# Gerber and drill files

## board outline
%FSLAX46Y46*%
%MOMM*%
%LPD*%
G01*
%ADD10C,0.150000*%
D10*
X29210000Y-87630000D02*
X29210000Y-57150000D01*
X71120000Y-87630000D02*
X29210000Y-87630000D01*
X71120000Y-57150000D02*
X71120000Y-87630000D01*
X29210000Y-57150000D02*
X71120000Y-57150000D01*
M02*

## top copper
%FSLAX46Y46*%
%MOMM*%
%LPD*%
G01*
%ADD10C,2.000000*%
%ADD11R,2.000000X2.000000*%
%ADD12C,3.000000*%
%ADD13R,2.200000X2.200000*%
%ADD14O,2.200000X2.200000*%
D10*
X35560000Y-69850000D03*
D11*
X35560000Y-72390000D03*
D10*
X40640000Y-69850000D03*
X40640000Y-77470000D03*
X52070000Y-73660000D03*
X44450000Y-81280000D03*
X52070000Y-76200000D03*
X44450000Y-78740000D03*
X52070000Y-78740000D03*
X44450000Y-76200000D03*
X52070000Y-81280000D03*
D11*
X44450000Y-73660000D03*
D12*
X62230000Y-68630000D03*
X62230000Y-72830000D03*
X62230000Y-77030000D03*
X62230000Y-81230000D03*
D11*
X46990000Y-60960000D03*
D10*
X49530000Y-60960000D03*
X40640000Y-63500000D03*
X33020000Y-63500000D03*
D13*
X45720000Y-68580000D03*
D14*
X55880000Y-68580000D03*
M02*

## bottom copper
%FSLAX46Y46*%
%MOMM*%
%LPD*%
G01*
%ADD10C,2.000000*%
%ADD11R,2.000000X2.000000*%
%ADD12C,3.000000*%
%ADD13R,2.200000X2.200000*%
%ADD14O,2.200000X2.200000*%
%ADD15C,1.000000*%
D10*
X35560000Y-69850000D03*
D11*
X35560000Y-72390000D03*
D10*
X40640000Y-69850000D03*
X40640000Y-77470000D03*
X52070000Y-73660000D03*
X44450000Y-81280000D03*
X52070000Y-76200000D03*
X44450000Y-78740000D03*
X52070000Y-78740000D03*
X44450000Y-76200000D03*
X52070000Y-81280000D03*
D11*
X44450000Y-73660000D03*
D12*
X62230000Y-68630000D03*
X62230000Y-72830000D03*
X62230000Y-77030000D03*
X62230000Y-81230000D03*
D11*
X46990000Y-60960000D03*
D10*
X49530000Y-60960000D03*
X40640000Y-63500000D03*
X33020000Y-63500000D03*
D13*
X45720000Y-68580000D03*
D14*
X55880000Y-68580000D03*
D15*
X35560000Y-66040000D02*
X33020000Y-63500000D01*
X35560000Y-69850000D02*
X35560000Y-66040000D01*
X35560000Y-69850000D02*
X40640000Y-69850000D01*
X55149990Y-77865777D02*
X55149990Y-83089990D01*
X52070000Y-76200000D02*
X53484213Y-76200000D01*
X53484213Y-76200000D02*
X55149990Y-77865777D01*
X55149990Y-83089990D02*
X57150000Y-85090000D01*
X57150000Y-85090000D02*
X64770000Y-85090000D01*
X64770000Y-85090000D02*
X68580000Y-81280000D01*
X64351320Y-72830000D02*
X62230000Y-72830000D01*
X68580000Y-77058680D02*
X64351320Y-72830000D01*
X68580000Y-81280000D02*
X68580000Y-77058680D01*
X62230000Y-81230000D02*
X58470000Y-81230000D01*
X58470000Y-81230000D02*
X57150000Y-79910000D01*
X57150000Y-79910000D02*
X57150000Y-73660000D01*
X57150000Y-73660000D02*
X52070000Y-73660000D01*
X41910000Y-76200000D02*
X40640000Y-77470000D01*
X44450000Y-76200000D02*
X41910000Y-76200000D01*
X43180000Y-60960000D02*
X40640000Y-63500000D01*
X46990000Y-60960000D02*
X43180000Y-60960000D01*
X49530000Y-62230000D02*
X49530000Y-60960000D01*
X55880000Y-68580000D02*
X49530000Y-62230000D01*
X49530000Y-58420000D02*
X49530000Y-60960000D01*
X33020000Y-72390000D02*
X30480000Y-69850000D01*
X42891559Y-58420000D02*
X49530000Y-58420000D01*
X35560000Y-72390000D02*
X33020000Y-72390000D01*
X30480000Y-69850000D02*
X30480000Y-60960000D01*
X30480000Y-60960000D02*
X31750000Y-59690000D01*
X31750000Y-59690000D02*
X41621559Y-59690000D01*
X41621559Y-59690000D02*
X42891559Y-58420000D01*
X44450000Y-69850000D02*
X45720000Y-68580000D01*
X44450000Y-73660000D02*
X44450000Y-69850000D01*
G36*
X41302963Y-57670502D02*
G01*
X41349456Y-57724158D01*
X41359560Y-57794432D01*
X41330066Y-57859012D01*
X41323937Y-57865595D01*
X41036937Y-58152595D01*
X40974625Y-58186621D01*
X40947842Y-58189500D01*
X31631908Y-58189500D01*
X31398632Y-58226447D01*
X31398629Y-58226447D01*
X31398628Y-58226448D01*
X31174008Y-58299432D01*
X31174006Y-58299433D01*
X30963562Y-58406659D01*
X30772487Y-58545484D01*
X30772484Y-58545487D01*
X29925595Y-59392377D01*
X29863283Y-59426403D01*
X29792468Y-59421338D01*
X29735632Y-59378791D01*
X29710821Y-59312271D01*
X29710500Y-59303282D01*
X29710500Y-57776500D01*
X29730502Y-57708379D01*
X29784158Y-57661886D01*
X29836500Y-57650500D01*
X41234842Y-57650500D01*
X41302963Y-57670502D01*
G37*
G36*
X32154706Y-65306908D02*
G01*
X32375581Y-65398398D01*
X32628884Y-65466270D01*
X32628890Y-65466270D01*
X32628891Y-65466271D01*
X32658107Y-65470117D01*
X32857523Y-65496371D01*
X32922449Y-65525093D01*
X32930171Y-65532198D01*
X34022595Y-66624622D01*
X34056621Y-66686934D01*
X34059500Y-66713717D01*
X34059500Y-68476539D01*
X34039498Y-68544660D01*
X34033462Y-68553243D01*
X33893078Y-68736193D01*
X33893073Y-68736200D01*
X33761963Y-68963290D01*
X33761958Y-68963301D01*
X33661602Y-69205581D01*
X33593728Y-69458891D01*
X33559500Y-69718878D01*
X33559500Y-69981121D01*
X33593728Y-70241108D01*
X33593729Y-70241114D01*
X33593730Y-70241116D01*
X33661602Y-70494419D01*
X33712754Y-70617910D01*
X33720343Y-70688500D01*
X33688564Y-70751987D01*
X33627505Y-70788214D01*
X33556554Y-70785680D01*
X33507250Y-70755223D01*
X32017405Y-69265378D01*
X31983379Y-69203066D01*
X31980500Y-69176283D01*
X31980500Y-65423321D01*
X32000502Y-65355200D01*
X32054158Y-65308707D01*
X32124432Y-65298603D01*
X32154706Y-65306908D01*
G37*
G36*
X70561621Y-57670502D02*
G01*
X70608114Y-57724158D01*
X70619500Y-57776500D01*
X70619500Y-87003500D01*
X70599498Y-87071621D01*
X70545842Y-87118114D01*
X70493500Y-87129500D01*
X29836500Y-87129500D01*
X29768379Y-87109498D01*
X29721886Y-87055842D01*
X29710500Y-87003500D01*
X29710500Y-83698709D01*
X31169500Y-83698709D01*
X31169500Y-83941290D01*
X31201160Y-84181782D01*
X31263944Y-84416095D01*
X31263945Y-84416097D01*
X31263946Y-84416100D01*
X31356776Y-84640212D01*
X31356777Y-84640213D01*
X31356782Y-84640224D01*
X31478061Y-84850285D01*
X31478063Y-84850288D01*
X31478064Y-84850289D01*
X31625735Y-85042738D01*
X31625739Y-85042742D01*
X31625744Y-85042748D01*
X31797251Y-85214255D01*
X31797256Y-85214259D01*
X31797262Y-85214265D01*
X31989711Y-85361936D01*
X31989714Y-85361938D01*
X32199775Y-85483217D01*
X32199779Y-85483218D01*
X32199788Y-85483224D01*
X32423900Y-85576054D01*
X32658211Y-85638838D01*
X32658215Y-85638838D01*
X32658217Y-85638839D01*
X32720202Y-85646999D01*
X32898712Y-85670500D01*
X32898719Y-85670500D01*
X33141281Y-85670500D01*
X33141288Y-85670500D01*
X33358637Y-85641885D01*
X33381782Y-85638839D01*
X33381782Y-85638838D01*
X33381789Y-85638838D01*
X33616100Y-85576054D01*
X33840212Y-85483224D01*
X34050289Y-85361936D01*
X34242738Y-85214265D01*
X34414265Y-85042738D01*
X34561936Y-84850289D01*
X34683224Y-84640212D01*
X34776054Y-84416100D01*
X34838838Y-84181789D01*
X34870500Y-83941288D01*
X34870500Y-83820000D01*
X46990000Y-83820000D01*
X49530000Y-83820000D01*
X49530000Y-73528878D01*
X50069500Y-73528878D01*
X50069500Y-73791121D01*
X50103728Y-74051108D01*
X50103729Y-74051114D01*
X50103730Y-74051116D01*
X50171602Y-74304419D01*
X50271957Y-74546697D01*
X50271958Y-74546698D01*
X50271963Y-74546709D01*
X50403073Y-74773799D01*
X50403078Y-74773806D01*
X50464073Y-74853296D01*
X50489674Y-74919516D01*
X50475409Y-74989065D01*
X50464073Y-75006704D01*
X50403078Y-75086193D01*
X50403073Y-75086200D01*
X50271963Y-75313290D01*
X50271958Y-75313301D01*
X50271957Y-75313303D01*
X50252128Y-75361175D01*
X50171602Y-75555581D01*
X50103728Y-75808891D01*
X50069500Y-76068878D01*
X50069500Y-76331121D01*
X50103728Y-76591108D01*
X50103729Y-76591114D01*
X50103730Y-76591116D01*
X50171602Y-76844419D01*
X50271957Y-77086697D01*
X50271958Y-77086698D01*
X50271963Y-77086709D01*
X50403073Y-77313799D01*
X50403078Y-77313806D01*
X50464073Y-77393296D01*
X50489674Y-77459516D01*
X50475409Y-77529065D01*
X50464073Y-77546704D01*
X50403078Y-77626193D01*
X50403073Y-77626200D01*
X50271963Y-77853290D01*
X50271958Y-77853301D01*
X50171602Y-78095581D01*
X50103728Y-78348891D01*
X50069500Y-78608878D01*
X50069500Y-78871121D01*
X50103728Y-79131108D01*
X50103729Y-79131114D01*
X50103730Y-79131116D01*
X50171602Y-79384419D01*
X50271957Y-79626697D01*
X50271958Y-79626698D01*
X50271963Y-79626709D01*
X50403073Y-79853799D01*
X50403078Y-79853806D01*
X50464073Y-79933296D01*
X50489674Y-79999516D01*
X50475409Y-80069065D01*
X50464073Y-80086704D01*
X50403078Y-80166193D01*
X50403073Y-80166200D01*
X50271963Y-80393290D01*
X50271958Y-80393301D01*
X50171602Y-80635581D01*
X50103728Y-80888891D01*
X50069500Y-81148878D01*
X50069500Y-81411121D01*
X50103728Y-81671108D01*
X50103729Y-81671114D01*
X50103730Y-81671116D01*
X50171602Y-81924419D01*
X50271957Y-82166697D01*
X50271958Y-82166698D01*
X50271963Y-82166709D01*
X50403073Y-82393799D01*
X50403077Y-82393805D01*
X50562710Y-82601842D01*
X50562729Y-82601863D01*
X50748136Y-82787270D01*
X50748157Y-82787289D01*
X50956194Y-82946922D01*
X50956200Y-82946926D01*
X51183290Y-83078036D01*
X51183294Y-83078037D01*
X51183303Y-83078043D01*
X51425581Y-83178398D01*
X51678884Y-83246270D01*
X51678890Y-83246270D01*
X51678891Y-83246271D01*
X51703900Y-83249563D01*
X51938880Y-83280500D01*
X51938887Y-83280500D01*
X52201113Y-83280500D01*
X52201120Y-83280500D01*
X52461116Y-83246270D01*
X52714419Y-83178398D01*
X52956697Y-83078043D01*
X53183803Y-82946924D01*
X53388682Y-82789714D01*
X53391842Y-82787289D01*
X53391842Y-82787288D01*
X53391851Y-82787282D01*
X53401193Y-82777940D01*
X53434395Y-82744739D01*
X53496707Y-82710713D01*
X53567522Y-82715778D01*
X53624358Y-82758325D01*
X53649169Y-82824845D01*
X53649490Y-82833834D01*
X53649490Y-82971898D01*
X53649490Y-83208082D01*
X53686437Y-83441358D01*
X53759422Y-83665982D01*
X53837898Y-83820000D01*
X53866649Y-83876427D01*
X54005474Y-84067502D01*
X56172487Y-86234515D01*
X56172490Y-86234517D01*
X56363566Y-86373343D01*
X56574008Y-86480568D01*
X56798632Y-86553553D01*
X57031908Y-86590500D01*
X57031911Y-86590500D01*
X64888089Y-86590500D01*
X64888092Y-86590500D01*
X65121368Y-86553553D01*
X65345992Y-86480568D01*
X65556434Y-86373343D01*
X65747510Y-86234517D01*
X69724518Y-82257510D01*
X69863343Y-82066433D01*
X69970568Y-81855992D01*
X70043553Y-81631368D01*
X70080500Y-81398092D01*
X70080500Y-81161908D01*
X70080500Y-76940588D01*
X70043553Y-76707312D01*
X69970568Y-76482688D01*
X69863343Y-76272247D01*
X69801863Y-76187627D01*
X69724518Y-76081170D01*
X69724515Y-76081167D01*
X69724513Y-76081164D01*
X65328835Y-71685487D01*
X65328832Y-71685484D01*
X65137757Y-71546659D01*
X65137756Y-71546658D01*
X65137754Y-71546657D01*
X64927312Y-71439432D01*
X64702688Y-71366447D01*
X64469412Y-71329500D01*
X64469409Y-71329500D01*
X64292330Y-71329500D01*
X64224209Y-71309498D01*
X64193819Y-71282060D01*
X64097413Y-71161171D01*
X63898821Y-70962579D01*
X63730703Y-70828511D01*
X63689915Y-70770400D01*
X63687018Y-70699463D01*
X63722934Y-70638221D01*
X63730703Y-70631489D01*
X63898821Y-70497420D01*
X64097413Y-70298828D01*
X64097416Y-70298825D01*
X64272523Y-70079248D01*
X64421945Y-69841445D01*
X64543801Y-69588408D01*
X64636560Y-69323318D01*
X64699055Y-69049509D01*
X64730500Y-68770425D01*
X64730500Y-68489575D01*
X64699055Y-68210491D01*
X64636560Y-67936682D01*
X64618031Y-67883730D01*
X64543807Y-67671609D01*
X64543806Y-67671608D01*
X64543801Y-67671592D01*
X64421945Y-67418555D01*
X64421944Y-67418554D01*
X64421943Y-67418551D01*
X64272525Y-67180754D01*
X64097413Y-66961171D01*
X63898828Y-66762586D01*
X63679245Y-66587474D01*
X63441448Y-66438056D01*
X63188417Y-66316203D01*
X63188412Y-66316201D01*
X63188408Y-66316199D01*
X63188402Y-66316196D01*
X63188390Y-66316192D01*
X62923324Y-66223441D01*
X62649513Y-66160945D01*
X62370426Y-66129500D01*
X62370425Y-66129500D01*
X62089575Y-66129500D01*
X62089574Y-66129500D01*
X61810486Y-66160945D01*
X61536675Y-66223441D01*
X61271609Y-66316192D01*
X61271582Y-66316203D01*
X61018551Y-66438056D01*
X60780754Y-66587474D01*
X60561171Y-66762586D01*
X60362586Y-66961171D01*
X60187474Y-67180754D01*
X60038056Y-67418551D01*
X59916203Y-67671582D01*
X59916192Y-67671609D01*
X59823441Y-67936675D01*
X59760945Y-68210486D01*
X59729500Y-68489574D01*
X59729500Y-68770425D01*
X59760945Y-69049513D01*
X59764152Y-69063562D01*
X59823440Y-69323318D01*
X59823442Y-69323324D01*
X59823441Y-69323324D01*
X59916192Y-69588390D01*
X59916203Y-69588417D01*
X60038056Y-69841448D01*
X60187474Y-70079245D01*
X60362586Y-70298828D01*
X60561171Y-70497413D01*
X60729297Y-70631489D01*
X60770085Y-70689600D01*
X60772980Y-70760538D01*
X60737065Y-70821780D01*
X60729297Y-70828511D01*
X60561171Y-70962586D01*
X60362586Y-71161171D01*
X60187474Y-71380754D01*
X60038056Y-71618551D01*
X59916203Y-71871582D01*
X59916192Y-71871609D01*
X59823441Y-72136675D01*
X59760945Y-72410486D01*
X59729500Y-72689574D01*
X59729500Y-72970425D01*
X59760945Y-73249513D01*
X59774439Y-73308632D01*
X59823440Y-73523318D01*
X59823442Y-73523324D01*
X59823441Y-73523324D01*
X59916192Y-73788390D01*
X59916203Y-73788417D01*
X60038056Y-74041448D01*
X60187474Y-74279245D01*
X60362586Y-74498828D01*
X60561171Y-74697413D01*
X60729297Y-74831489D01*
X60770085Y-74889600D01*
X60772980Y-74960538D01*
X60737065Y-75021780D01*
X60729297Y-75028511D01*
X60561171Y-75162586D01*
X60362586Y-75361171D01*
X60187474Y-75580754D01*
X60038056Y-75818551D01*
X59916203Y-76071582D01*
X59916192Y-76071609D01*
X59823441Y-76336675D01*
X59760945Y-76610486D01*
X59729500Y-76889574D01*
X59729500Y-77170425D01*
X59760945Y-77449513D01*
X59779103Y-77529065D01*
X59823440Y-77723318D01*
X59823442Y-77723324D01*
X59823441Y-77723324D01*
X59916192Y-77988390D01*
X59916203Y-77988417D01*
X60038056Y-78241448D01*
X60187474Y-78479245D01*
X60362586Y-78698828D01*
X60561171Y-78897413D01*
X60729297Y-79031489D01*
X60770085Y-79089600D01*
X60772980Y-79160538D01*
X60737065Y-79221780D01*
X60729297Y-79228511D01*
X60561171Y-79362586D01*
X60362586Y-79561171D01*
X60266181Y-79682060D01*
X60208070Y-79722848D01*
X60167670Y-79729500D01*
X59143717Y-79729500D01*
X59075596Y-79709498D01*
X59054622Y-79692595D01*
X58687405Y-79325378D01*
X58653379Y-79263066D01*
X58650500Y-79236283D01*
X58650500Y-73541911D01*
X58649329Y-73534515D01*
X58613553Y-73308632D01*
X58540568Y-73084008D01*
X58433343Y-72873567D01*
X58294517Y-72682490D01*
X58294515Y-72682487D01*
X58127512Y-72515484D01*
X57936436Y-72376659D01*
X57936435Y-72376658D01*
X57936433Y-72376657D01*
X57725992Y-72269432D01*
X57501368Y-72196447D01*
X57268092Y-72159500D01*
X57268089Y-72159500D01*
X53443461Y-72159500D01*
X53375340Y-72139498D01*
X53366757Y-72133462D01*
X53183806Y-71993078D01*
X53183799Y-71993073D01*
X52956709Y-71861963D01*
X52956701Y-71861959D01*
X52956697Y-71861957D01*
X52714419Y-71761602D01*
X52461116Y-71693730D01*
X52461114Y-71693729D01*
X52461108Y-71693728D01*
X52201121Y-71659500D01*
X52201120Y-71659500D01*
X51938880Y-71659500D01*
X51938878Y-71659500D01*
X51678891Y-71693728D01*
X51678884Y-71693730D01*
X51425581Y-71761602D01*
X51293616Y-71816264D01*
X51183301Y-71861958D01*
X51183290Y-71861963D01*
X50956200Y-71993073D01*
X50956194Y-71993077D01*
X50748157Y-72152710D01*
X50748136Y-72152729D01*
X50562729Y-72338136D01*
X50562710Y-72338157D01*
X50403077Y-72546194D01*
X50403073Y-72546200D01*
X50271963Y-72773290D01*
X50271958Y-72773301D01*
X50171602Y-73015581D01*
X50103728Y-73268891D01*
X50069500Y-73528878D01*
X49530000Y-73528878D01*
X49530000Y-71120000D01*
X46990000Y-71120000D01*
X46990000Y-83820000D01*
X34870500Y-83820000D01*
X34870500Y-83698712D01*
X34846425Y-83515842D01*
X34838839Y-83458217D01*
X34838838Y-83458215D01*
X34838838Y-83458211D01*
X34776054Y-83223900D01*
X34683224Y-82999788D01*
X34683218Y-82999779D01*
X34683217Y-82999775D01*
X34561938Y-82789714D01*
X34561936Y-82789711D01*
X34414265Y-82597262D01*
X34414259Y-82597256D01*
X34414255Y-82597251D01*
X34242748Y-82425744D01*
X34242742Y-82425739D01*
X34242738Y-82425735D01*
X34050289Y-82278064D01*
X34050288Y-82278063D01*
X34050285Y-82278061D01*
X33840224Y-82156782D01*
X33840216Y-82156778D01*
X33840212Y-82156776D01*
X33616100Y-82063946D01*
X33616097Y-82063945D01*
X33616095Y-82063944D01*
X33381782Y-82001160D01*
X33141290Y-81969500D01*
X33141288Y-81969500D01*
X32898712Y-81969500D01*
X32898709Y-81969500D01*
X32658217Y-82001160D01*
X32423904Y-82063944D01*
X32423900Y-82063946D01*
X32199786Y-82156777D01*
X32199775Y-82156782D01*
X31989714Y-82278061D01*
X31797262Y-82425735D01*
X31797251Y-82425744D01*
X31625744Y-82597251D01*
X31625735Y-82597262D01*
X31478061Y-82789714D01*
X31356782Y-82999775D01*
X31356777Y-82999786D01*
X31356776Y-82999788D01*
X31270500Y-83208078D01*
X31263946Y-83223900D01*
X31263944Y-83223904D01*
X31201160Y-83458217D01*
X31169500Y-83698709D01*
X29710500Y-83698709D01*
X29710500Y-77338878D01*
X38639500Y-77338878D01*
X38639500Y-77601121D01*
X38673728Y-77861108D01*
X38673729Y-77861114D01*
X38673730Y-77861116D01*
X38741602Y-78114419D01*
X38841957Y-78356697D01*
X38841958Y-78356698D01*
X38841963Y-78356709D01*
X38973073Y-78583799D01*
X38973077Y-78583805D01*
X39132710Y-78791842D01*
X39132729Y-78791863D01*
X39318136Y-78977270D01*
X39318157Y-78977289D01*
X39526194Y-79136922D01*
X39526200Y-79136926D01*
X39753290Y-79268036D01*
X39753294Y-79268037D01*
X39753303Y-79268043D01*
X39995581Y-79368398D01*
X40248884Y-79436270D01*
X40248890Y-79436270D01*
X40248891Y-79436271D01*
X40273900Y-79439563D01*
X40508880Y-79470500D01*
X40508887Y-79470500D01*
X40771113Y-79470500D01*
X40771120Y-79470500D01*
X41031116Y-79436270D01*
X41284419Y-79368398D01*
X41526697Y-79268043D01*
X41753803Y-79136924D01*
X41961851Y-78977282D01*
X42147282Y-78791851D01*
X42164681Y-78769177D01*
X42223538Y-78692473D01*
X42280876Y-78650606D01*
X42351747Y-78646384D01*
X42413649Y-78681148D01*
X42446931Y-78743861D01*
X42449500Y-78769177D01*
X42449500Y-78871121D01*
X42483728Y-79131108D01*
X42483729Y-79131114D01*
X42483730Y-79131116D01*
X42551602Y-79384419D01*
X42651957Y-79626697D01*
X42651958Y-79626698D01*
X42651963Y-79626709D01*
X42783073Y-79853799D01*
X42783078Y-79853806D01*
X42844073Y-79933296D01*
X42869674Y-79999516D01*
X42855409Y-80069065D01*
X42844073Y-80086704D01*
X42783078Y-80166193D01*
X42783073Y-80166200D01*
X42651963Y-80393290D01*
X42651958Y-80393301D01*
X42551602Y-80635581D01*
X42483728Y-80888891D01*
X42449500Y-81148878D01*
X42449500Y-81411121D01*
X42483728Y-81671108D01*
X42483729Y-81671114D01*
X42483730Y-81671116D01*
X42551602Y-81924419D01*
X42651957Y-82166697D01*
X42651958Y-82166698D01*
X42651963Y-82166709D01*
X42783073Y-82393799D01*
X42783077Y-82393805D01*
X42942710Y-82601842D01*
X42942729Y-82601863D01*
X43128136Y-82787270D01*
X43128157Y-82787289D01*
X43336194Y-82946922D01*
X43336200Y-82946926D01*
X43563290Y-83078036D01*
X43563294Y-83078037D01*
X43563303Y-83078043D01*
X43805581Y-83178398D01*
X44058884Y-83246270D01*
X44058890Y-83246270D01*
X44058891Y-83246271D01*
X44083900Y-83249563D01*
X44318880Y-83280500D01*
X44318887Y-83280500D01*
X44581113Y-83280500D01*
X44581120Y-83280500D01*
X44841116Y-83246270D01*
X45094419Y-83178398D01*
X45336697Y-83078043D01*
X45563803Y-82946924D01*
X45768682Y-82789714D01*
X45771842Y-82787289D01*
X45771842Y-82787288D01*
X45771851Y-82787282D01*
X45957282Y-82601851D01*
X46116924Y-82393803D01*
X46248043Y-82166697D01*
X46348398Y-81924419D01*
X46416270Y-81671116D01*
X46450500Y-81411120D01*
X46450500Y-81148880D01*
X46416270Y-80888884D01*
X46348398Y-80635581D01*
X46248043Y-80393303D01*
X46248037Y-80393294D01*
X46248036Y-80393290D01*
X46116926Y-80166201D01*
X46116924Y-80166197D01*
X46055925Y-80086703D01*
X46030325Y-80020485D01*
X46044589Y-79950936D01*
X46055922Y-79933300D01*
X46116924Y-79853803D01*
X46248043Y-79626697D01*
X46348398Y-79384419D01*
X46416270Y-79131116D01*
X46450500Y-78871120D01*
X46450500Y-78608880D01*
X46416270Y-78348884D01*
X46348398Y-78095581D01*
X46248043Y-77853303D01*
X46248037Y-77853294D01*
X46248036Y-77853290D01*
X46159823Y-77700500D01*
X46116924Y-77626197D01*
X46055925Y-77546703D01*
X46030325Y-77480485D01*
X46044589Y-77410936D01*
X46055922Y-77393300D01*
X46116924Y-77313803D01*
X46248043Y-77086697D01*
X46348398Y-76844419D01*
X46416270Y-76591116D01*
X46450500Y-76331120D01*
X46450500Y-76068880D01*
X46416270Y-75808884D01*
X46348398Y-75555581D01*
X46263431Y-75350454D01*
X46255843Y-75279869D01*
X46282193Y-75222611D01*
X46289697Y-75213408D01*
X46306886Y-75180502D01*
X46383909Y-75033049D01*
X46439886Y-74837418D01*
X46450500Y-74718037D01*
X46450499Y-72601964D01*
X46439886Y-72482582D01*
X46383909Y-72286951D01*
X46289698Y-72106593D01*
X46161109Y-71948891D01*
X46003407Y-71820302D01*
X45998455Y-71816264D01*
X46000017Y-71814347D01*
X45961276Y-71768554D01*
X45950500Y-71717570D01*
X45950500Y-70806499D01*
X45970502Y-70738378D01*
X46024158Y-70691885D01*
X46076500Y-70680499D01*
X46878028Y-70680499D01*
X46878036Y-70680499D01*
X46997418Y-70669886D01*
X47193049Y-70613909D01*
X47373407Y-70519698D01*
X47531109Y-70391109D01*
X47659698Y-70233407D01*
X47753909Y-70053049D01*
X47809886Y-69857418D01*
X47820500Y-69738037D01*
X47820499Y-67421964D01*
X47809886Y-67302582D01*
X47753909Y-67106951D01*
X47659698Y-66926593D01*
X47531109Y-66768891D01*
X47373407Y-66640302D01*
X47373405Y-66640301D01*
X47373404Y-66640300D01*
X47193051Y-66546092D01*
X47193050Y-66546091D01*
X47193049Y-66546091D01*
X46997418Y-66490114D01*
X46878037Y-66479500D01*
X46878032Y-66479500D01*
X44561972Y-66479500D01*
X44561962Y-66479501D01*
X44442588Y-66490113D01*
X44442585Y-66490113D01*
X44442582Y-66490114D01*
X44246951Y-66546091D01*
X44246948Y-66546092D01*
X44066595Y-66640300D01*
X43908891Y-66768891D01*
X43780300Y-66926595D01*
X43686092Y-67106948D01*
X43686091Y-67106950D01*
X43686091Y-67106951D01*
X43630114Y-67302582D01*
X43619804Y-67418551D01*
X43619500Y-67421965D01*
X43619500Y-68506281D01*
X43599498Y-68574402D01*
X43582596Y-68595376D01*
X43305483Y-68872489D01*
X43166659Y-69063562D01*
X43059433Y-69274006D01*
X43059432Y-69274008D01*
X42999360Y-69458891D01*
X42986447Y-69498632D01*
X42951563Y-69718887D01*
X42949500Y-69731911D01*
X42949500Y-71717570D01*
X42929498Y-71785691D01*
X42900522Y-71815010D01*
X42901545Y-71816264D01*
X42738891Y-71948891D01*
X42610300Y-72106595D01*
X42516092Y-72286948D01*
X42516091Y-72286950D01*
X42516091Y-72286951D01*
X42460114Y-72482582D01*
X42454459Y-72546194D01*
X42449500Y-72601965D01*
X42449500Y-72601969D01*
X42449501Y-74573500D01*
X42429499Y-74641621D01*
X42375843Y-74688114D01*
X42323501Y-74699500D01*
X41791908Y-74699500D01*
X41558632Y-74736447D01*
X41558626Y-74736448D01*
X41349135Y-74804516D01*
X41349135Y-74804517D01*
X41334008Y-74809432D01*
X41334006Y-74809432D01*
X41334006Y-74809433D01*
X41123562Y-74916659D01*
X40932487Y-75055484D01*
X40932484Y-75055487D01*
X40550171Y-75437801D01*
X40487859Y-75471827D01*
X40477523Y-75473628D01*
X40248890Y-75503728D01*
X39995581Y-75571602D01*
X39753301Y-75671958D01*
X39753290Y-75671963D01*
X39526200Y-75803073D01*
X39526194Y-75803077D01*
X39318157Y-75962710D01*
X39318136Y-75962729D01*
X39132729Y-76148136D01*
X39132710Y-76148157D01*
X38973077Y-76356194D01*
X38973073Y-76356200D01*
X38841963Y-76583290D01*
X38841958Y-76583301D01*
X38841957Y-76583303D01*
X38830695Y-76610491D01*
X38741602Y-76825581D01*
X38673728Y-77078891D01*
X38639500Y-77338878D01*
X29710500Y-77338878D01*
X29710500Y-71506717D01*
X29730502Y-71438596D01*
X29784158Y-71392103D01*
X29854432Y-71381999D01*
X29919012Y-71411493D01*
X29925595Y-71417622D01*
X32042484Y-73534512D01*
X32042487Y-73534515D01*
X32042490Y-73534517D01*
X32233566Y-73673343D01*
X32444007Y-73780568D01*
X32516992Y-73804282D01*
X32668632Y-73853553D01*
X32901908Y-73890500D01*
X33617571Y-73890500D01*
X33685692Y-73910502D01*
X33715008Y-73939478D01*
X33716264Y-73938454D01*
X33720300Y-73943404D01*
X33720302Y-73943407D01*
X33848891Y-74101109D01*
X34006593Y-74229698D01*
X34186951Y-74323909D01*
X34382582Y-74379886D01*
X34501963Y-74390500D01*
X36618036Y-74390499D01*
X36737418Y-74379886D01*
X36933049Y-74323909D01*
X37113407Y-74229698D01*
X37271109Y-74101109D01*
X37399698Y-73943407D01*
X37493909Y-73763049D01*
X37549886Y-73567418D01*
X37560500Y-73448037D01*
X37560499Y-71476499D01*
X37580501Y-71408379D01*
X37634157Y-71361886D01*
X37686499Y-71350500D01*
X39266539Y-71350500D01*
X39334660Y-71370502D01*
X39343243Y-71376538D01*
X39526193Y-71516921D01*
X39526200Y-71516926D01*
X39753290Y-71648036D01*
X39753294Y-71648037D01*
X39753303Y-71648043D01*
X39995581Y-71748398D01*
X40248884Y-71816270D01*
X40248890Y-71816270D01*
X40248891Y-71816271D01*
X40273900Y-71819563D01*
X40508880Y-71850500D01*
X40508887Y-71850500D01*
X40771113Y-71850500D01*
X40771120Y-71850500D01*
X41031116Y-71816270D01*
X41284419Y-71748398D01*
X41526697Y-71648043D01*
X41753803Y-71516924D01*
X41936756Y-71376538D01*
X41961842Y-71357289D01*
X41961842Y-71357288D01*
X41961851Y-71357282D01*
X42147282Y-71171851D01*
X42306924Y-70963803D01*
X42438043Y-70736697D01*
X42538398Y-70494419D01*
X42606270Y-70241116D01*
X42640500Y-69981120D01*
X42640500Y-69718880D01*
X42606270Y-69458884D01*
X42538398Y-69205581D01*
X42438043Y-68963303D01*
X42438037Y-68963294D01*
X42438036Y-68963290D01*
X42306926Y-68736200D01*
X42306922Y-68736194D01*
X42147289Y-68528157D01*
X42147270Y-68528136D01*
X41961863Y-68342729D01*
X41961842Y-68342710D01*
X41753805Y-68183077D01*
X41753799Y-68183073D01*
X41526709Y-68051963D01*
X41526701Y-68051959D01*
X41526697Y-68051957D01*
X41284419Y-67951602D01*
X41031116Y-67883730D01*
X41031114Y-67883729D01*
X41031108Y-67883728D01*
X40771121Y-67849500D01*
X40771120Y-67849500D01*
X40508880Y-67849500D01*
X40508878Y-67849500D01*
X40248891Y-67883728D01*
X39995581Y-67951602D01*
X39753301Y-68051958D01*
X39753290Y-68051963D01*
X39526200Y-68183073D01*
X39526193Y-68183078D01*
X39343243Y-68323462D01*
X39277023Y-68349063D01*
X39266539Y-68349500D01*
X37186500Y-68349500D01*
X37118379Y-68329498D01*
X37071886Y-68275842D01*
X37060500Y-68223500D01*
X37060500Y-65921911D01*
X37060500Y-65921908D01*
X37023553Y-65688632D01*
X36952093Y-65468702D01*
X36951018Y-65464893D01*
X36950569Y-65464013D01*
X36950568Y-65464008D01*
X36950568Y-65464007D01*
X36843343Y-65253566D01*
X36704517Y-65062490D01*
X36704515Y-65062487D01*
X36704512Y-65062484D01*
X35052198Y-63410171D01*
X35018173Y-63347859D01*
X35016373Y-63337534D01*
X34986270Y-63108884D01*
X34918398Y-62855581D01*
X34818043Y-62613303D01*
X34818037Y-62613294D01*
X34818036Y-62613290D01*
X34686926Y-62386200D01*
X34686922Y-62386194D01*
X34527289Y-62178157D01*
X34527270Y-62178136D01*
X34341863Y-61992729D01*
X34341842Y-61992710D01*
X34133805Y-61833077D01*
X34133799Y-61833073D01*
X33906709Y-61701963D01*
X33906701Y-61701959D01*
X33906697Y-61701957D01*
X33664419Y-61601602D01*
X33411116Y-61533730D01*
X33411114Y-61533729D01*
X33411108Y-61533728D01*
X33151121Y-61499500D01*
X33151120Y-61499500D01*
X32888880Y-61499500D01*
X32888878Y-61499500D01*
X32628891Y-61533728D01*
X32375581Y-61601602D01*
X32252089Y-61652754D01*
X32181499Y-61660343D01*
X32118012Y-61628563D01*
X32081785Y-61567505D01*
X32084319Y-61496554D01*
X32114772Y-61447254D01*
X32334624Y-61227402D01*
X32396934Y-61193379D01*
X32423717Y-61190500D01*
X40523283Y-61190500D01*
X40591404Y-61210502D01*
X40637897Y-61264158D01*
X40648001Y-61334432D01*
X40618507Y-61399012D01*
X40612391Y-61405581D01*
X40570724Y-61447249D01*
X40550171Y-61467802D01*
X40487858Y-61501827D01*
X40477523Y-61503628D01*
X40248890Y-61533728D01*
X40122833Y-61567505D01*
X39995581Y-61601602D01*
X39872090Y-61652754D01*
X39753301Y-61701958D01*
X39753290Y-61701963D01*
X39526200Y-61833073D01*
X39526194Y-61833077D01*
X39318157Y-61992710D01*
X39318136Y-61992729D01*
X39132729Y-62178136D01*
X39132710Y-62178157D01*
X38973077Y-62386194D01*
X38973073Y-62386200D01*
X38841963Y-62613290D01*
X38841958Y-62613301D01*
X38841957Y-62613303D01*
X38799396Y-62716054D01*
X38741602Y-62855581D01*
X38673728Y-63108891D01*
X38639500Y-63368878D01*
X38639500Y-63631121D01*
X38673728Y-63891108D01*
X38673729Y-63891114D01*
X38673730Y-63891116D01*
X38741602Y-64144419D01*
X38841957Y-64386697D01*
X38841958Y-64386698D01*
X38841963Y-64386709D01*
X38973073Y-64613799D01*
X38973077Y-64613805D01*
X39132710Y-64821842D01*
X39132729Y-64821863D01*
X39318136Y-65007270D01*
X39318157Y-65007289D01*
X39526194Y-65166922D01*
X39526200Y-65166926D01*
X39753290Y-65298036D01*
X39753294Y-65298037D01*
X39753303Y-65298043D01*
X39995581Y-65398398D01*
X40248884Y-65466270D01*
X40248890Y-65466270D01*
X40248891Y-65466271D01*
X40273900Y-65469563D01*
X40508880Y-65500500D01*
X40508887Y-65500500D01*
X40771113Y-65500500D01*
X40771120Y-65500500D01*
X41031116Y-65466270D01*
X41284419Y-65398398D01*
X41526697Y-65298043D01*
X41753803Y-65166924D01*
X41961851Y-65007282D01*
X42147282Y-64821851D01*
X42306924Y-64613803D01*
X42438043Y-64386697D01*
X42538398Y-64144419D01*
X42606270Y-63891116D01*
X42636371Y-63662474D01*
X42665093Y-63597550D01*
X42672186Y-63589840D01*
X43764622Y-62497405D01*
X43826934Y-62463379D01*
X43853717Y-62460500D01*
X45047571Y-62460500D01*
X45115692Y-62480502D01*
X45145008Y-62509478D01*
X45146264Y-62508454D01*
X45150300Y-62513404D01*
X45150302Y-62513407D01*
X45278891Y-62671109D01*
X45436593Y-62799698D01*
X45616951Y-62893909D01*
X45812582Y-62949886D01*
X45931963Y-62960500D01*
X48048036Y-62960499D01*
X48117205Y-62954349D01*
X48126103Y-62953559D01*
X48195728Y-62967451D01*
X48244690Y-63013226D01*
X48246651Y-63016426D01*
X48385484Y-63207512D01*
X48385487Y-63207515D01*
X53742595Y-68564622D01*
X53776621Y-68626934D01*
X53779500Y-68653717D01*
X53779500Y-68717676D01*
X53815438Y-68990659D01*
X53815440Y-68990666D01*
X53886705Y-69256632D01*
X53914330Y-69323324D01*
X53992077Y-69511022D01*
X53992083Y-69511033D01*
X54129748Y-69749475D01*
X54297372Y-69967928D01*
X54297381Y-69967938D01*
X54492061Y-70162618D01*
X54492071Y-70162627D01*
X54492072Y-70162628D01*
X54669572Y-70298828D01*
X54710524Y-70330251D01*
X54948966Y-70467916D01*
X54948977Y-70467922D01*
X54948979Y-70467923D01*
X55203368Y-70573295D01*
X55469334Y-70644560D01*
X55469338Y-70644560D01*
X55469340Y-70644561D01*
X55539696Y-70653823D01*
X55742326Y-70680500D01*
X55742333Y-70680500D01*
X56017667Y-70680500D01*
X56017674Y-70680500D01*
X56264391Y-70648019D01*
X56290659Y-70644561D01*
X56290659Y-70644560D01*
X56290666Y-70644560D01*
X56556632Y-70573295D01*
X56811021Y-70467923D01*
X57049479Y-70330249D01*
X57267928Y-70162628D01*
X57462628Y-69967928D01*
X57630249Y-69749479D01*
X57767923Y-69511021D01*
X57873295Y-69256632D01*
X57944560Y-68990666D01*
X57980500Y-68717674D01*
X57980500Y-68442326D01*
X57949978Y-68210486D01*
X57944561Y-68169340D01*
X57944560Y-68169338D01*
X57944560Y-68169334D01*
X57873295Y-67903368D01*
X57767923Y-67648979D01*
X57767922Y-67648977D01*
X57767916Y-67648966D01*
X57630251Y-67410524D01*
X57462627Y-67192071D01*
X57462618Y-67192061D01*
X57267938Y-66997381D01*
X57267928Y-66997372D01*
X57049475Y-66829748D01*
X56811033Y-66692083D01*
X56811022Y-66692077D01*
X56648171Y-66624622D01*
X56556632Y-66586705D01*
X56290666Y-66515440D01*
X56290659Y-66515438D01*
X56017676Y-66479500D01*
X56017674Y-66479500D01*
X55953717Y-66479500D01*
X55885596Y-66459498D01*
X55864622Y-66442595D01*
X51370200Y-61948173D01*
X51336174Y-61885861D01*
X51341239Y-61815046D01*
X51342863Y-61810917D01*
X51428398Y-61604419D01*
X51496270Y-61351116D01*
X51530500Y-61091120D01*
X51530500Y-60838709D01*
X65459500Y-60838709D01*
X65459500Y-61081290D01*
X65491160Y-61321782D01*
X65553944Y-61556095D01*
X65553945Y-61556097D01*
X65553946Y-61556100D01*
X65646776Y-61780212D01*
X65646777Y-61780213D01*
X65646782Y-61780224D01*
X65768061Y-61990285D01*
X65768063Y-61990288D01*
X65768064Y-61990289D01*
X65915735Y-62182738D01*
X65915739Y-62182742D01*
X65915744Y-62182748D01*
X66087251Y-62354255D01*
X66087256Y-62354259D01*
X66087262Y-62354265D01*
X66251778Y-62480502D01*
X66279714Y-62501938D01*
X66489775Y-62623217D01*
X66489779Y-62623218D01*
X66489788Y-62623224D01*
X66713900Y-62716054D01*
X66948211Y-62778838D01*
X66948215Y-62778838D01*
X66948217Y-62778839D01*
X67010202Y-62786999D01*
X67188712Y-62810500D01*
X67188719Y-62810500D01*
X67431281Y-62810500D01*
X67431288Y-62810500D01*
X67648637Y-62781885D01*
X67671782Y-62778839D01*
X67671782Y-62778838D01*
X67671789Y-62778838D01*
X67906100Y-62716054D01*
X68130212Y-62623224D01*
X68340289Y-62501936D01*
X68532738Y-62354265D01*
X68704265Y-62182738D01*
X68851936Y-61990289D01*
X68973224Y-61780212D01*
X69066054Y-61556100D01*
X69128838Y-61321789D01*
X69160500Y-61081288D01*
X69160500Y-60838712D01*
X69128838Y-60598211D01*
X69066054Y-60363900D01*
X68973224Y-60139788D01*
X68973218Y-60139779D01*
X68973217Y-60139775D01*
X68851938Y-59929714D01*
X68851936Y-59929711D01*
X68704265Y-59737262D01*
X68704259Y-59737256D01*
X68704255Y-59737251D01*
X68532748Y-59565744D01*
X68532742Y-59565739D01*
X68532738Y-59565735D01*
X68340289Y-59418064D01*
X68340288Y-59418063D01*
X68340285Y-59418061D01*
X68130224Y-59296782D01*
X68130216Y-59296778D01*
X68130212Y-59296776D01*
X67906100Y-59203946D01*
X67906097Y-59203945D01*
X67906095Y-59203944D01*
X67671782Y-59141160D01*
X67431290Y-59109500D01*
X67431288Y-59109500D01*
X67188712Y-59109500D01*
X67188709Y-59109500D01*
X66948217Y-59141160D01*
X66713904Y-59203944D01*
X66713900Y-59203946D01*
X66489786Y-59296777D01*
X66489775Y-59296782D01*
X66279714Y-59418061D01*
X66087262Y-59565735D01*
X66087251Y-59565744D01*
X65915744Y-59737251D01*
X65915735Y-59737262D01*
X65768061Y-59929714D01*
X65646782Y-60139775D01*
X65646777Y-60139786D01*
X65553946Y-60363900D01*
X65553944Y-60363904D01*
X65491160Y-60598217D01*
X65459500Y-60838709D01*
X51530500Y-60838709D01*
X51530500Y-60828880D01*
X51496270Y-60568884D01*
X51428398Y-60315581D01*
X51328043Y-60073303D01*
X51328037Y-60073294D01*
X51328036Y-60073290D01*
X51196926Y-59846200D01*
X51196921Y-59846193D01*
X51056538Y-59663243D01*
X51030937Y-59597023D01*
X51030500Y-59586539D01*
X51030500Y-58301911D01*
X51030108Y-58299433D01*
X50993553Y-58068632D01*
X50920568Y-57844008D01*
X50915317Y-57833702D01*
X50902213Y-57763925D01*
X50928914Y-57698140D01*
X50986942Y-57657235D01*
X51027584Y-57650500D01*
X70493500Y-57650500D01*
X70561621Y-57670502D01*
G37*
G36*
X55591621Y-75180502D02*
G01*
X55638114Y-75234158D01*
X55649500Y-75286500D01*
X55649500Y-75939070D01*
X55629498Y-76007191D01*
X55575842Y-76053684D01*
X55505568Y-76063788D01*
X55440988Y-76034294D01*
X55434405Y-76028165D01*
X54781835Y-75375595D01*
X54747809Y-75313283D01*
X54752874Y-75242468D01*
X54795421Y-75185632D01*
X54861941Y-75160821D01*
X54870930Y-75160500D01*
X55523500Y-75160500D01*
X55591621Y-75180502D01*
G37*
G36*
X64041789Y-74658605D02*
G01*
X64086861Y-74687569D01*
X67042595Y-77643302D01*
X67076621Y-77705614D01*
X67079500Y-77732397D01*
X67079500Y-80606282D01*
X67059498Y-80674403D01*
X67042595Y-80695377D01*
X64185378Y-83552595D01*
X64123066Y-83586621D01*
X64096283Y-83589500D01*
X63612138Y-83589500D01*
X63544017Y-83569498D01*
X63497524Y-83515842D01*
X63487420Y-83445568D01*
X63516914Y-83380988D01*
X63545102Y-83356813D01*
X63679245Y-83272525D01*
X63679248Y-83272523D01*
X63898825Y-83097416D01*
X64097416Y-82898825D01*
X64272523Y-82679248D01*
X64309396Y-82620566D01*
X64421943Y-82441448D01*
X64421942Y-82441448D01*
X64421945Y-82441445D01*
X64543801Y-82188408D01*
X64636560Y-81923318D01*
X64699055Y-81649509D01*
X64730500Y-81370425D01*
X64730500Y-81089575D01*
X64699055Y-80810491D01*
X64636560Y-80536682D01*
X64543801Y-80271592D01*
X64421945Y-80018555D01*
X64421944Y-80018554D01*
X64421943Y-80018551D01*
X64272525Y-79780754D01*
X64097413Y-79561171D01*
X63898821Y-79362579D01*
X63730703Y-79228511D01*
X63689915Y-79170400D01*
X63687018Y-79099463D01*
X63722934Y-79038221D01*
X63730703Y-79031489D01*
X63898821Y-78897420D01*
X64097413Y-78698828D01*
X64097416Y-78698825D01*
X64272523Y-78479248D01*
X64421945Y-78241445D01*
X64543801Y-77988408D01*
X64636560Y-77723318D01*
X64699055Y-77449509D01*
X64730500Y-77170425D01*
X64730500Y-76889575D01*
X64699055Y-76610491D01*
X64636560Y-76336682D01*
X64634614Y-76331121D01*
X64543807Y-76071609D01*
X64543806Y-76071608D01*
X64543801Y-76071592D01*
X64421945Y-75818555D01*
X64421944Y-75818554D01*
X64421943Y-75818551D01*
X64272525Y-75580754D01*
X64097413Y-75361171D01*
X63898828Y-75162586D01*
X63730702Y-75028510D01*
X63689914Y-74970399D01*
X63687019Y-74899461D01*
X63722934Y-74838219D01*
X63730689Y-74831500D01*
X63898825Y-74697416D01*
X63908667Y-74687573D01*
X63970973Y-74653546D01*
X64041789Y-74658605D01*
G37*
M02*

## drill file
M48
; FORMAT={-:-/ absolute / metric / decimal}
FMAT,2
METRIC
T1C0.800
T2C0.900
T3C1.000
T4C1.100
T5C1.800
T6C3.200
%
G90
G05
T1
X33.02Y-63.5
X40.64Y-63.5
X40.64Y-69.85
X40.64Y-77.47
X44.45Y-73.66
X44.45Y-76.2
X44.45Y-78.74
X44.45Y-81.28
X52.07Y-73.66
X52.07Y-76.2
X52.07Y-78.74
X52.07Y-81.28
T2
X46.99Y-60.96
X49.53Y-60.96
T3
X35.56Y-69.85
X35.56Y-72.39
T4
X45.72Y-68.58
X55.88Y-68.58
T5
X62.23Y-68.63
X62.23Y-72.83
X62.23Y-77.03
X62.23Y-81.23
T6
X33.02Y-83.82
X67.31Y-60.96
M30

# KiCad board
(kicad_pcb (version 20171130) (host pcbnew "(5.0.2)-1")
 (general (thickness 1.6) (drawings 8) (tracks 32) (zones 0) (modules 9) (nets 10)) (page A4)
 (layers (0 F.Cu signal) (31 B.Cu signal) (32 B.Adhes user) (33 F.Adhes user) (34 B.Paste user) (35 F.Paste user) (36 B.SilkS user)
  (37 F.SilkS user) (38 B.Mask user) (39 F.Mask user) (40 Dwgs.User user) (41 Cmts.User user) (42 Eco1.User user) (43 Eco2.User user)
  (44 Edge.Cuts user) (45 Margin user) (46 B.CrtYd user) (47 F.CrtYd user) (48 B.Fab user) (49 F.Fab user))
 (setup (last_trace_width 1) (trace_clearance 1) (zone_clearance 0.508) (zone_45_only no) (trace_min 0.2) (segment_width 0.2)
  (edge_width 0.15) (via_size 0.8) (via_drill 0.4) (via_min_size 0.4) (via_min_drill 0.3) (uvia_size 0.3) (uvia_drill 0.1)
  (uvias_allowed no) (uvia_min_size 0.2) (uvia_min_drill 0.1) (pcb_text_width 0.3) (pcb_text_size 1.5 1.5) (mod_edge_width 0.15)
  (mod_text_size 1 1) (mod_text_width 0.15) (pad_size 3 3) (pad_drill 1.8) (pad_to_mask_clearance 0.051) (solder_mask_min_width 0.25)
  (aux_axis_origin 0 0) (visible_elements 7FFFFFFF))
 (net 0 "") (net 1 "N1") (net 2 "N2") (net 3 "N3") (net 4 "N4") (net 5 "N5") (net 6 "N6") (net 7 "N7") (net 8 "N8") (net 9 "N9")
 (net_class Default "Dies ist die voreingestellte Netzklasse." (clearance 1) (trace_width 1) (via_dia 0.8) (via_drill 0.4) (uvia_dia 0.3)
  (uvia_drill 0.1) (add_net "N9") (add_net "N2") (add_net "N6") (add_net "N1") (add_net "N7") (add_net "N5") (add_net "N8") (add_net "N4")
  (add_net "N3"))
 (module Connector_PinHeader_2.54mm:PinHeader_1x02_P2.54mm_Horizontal (layer F.Cu) (at 35.56 72.39 180)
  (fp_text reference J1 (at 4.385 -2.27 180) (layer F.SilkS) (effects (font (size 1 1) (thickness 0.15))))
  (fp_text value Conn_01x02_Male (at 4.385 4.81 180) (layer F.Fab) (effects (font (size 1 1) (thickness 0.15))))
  (pad 2 thru_hole circle (at 0 2.54 180) (size 2 2) (drill 1) (layers *.Cu *.Mask) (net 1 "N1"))
  (pad 1 thru_hole rect (at 0 0 180) (size 2 2) (drill 1) (layers *.Cu *.Mask) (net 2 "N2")))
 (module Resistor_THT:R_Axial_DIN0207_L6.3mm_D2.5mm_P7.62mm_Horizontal (layer F.Cu) (at 40.64 77.47 90)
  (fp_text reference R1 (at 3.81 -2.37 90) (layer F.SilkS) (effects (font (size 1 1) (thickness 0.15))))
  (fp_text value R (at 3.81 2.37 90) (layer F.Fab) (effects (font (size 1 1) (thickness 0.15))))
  (pad 2 thru_hole circle (at 7.62 0 90) (size 2 2) (drill 0.8) (layers *.Cu *.Mask) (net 1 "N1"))
  (pad 1 thru_hole circle (at 0 0 90) (size 2 2) (drill 0.8) (layers *.Cu *.Mask) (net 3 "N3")))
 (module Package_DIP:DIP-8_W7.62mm (layer F.Cu) (at 44.45 73.66)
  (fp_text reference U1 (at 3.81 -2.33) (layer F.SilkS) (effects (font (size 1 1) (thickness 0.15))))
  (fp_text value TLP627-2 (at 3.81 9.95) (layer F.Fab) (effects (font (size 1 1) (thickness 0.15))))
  (pad 8 thru_hole circle (at 7.62 0) (size 2 2) (drill 0.8) (layers *.Cu *.Mask) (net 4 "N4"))
  (pad 4 thru_hole circle (at 0 7.62) (size 2 2) (drill 0.8) (layers *.Cu *.Mask))
  (pad 7 thru_hole circle (at 7.62 2.54) (size 2 2) (drill 0.8) (layers *.Cu *.Mask) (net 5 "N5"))
  (pad 3 thru_hole circle (at 0 5.08) (size 2 2) (drill 0.8) (layers *.Cu *.Mask))
  (pad 6 thru_hole circle (at 7.62 5.08) (size 2 2) (drill 0.8) (layers *.Cu *.Mask))
  (pad 2 thru_hole circle (at 0 2.54) (size 2 2) (drill 0.8) (layers *.Cu *.Mask) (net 3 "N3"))
  (pad 5 thru_hole circle (at 7.62 7.62) (size 2 2) (drill 0.8) (layers *.Cu *.Mask))
  (pad 1 thru_hole rect (at 0 0) (size 2 2) (drill 0.8) (layers *.Cu *.Mask) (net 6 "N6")))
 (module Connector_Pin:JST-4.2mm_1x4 (layer F.Cu) (at 62.23 74.93 270)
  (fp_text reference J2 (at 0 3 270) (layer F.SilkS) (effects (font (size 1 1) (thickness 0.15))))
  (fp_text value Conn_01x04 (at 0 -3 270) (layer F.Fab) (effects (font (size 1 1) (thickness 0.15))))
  (pad 1 thru_hole circle (at -6.3 0 270) (size 3 3) (drill 1.8) (layers *.Cu *.Mask) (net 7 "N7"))
  (pad 2 thru_hole circle (at -2.1 0 270) (size 3 3) (drill 1.8) (layers *.Cu *.Mask) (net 5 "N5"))
  (pad 3 thru_hole circle (at 2.1 0 270) (size 3 3) (drill 1.8) (layers *.Cu *.Mask) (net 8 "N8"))
  (pad 4 thru_hole circle (at 6.3 0 270) (size 3 3) (drill 1.8) (layers *.Cu *.Mask) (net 4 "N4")))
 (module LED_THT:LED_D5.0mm (layer F.Cu) (at 46.99 60.96)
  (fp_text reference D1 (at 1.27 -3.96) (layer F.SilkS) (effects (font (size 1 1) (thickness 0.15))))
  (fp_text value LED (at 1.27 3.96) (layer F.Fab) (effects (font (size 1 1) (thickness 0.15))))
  (pad 1 thru_hole rect (at 0 0) (size 2 2) (drill 0.9) (layers *.Cu *.Mask) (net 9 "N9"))
  (pad 2 thru_hole circle (at 2.54 0) (size 2 2) (drill 0.9) (layers *.Cu *.Mask) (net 2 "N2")))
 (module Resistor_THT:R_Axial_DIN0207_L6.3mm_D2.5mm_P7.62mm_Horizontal (layer F.Cu) (at 40.64 63.5 180)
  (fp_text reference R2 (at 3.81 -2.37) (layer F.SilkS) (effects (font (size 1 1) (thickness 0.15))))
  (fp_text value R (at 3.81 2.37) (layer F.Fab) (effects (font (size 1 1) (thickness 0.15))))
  (pad 1 thru_hole circle (at 0 0 180) (size 2 2) (drill 0.8) (layers *.Cu *.Mask) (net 9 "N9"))
  (pad 2 thru_hole circle (at 7.62 0 180) (size 2 2) (drill 0.8) (layers *.Cu *.Mask) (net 1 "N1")))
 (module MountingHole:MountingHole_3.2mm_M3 (layer F.Cu) (at 33.02 83.82)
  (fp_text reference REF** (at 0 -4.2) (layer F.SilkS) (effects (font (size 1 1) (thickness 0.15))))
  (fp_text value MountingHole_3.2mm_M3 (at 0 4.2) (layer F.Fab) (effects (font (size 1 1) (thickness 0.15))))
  (pad 1 np_thru_hole circle (at 0 0) (size 3.2 3.2) (drill 3.2) (layers *.Cu *.Mask)))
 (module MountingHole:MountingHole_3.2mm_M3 (layer F.Cu) (at 67.31 60.96)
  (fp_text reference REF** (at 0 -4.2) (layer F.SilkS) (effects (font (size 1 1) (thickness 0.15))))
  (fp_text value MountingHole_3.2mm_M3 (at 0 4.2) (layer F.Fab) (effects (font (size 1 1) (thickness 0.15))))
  (pad 1 np_thru_hole circle (at 0 0) (size 3.2 3.2) (drill 3.2) (layers *.Cu *.Mask)))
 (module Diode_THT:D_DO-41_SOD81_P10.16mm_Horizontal (layer F.Cu) (at 45.72 68.58)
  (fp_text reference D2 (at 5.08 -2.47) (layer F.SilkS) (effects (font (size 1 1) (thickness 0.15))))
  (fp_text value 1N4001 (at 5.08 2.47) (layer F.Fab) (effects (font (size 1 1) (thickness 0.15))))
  (pad 1 thru_hole rect (at 0 0) (size 2.2 2.2) (drill 1.1) (layers *.Cu *.Mask) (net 6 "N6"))
  (pad 2 thru_hole oval (at 10.16 0) (size 2.2 2.2) (drill 1.1) (layers *.Cu *.Mask) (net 2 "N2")))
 (gr_line (start 29.21 87.63) (end 29.21 57.15) (layer Edge.Cuts) (width 0.15))
 (gr_line (start 71.12 87.63) (end 29.21 87.63) (layer Edge.Cuts) (width 0.15))
 (gr_line (start 71.12 57.15) (end 71.12 87.63) (layer Edge.Cuts) (width 0.15))
 (gr_line (start 29.21 57.15) (end 71.12 57.15) (layer Edge.Cuts) (width 0.15))
 (segment (start 35.56 66.04) (end 33.02 63.5) (width 1) (layer B.Cu) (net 1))
 (segment (start 35.56 69.85) (end 35.56 66.04) (width 1) (layer B.Cu) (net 1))
 (segment (start 35.56 69.85) (end 40.64 69.85) (width 1) (layer B.Cu) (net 1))
 (segment (start 55.14999 77.865777) (end 55.14999 83.08999) (width 1) (layer B.Cu) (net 5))
 (segment (start 52.07 76.2) (end 53.484213 76.2) (width 1) (layer B.Cu) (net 5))
 (segment (start 53.484213 76.2) (end 55.14999 77.865777) (width 1) (layer B.Cu) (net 5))
 (segment (start 55.14999 83.08999) (end 57.15 85.09) (width 1) (layer B.Cu) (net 5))
 (segment (start 57.15 85.09) (end 64.77 85.09) (width 1) (layer B.Cu) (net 5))
 (segment (start 64.77 85.09) (end 68.58 81.28) (width 1) (layer B.Cu) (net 5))
 (segment (start 64.35132 72.83) (end 62.23 72.83) (width 1) (layer B.Cu) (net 5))
 (segment (start 68.58 77.05868) (end 64.35132 72.83) (width 1) (layer B.Cu) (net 5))
 (segment (start 68.58 81.28) (end 68.58 77.05868) (width 1) (layer B.Cu) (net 5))
 (segment (start 62.23 81.23) (end 58.47 81.23) (width 1) (layer B.Cu) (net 4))
 (segment (start 58.47 81.23) (end 57.15 79.91) (width 1) (layer B.Cu) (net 4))
 (segment (start 57.15 79.91) (end 57.15 73.66) (width 1) (layer B.Cu) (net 4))
 (segment (start 57.15 73.66) (end 52.07 73.66) (width 1) (layer B.Cu) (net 4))
 (segment (start 41.91 76.2) (end 40.64 77.47) (width 1) (layer B.Cu) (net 3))
 (segment (start 44.45 76.2) (end 41.91 76.2) (width 1) (layer B.Cu) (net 3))
 (segment (start 43.18 60.96) (end 40.64 63.5) (width 1) (layer B.Cu) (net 9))
 (segment (start 46.99 60.96) (end 43.18 60.96) (width 1) (layer B.Cu) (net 9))
 (segment (start 49.53 62.23) (end 49.53 60.96) (width 1) (layer B.Cu) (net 2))
 (segment (start 55.88 68.58) (end 49.53 62.23) (width 1) (layer B.Cu) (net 2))
 (segment (start 49.53 58.42) (end 49.53 60.96) (width 1) (layer B.Cu) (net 2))
 (segment (start 33.02 72.39) (end 30.48 69.85) (width 1) (layer B.Cu) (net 2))
 (segment (start 42.891559 58.42) (end 49.53 58.42) (width 1) (layer B.Cu) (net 2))
 (segment (start 35.56 72.39) (end 33.02 72.39) (width 1) (layer B.Cu) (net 2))
 (segment (start 30.48 69.85) (end 30.48 60.96) (width 1) (layer B.Cu) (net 2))
 (segment (start 30.48 60.96) (end 31.75 59.69) (width 1) (layer B.Cu) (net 2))
 (segment (start 31.75 59.69) (end 41.621559 59.69) (width 1) (layer B.Cu) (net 2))
 (segment (start 41.621559 59.69) (end 42.891559 58.42) (width 1) (layer B.Cu) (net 2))
 (segment (start 44.45 69.85) (end 45.72 68.58) (width 1) (layer B.Cu) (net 6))
 (segment (start 44.45 73.66) (end 44.45 69.85) (width 1) (layer B.Cu) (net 6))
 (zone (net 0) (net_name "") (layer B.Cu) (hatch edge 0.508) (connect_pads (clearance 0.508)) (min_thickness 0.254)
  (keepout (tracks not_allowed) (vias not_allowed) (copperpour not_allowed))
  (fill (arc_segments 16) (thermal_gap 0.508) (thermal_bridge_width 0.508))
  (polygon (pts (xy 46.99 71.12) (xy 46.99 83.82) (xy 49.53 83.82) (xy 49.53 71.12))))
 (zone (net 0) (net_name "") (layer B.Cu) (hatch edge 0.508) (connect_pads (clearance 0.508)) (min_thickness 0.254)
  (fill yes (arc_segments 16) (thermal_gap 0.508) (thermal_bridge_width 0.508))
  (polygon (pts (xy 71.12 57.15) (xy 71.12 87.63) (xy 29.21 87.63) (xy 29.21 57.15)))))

